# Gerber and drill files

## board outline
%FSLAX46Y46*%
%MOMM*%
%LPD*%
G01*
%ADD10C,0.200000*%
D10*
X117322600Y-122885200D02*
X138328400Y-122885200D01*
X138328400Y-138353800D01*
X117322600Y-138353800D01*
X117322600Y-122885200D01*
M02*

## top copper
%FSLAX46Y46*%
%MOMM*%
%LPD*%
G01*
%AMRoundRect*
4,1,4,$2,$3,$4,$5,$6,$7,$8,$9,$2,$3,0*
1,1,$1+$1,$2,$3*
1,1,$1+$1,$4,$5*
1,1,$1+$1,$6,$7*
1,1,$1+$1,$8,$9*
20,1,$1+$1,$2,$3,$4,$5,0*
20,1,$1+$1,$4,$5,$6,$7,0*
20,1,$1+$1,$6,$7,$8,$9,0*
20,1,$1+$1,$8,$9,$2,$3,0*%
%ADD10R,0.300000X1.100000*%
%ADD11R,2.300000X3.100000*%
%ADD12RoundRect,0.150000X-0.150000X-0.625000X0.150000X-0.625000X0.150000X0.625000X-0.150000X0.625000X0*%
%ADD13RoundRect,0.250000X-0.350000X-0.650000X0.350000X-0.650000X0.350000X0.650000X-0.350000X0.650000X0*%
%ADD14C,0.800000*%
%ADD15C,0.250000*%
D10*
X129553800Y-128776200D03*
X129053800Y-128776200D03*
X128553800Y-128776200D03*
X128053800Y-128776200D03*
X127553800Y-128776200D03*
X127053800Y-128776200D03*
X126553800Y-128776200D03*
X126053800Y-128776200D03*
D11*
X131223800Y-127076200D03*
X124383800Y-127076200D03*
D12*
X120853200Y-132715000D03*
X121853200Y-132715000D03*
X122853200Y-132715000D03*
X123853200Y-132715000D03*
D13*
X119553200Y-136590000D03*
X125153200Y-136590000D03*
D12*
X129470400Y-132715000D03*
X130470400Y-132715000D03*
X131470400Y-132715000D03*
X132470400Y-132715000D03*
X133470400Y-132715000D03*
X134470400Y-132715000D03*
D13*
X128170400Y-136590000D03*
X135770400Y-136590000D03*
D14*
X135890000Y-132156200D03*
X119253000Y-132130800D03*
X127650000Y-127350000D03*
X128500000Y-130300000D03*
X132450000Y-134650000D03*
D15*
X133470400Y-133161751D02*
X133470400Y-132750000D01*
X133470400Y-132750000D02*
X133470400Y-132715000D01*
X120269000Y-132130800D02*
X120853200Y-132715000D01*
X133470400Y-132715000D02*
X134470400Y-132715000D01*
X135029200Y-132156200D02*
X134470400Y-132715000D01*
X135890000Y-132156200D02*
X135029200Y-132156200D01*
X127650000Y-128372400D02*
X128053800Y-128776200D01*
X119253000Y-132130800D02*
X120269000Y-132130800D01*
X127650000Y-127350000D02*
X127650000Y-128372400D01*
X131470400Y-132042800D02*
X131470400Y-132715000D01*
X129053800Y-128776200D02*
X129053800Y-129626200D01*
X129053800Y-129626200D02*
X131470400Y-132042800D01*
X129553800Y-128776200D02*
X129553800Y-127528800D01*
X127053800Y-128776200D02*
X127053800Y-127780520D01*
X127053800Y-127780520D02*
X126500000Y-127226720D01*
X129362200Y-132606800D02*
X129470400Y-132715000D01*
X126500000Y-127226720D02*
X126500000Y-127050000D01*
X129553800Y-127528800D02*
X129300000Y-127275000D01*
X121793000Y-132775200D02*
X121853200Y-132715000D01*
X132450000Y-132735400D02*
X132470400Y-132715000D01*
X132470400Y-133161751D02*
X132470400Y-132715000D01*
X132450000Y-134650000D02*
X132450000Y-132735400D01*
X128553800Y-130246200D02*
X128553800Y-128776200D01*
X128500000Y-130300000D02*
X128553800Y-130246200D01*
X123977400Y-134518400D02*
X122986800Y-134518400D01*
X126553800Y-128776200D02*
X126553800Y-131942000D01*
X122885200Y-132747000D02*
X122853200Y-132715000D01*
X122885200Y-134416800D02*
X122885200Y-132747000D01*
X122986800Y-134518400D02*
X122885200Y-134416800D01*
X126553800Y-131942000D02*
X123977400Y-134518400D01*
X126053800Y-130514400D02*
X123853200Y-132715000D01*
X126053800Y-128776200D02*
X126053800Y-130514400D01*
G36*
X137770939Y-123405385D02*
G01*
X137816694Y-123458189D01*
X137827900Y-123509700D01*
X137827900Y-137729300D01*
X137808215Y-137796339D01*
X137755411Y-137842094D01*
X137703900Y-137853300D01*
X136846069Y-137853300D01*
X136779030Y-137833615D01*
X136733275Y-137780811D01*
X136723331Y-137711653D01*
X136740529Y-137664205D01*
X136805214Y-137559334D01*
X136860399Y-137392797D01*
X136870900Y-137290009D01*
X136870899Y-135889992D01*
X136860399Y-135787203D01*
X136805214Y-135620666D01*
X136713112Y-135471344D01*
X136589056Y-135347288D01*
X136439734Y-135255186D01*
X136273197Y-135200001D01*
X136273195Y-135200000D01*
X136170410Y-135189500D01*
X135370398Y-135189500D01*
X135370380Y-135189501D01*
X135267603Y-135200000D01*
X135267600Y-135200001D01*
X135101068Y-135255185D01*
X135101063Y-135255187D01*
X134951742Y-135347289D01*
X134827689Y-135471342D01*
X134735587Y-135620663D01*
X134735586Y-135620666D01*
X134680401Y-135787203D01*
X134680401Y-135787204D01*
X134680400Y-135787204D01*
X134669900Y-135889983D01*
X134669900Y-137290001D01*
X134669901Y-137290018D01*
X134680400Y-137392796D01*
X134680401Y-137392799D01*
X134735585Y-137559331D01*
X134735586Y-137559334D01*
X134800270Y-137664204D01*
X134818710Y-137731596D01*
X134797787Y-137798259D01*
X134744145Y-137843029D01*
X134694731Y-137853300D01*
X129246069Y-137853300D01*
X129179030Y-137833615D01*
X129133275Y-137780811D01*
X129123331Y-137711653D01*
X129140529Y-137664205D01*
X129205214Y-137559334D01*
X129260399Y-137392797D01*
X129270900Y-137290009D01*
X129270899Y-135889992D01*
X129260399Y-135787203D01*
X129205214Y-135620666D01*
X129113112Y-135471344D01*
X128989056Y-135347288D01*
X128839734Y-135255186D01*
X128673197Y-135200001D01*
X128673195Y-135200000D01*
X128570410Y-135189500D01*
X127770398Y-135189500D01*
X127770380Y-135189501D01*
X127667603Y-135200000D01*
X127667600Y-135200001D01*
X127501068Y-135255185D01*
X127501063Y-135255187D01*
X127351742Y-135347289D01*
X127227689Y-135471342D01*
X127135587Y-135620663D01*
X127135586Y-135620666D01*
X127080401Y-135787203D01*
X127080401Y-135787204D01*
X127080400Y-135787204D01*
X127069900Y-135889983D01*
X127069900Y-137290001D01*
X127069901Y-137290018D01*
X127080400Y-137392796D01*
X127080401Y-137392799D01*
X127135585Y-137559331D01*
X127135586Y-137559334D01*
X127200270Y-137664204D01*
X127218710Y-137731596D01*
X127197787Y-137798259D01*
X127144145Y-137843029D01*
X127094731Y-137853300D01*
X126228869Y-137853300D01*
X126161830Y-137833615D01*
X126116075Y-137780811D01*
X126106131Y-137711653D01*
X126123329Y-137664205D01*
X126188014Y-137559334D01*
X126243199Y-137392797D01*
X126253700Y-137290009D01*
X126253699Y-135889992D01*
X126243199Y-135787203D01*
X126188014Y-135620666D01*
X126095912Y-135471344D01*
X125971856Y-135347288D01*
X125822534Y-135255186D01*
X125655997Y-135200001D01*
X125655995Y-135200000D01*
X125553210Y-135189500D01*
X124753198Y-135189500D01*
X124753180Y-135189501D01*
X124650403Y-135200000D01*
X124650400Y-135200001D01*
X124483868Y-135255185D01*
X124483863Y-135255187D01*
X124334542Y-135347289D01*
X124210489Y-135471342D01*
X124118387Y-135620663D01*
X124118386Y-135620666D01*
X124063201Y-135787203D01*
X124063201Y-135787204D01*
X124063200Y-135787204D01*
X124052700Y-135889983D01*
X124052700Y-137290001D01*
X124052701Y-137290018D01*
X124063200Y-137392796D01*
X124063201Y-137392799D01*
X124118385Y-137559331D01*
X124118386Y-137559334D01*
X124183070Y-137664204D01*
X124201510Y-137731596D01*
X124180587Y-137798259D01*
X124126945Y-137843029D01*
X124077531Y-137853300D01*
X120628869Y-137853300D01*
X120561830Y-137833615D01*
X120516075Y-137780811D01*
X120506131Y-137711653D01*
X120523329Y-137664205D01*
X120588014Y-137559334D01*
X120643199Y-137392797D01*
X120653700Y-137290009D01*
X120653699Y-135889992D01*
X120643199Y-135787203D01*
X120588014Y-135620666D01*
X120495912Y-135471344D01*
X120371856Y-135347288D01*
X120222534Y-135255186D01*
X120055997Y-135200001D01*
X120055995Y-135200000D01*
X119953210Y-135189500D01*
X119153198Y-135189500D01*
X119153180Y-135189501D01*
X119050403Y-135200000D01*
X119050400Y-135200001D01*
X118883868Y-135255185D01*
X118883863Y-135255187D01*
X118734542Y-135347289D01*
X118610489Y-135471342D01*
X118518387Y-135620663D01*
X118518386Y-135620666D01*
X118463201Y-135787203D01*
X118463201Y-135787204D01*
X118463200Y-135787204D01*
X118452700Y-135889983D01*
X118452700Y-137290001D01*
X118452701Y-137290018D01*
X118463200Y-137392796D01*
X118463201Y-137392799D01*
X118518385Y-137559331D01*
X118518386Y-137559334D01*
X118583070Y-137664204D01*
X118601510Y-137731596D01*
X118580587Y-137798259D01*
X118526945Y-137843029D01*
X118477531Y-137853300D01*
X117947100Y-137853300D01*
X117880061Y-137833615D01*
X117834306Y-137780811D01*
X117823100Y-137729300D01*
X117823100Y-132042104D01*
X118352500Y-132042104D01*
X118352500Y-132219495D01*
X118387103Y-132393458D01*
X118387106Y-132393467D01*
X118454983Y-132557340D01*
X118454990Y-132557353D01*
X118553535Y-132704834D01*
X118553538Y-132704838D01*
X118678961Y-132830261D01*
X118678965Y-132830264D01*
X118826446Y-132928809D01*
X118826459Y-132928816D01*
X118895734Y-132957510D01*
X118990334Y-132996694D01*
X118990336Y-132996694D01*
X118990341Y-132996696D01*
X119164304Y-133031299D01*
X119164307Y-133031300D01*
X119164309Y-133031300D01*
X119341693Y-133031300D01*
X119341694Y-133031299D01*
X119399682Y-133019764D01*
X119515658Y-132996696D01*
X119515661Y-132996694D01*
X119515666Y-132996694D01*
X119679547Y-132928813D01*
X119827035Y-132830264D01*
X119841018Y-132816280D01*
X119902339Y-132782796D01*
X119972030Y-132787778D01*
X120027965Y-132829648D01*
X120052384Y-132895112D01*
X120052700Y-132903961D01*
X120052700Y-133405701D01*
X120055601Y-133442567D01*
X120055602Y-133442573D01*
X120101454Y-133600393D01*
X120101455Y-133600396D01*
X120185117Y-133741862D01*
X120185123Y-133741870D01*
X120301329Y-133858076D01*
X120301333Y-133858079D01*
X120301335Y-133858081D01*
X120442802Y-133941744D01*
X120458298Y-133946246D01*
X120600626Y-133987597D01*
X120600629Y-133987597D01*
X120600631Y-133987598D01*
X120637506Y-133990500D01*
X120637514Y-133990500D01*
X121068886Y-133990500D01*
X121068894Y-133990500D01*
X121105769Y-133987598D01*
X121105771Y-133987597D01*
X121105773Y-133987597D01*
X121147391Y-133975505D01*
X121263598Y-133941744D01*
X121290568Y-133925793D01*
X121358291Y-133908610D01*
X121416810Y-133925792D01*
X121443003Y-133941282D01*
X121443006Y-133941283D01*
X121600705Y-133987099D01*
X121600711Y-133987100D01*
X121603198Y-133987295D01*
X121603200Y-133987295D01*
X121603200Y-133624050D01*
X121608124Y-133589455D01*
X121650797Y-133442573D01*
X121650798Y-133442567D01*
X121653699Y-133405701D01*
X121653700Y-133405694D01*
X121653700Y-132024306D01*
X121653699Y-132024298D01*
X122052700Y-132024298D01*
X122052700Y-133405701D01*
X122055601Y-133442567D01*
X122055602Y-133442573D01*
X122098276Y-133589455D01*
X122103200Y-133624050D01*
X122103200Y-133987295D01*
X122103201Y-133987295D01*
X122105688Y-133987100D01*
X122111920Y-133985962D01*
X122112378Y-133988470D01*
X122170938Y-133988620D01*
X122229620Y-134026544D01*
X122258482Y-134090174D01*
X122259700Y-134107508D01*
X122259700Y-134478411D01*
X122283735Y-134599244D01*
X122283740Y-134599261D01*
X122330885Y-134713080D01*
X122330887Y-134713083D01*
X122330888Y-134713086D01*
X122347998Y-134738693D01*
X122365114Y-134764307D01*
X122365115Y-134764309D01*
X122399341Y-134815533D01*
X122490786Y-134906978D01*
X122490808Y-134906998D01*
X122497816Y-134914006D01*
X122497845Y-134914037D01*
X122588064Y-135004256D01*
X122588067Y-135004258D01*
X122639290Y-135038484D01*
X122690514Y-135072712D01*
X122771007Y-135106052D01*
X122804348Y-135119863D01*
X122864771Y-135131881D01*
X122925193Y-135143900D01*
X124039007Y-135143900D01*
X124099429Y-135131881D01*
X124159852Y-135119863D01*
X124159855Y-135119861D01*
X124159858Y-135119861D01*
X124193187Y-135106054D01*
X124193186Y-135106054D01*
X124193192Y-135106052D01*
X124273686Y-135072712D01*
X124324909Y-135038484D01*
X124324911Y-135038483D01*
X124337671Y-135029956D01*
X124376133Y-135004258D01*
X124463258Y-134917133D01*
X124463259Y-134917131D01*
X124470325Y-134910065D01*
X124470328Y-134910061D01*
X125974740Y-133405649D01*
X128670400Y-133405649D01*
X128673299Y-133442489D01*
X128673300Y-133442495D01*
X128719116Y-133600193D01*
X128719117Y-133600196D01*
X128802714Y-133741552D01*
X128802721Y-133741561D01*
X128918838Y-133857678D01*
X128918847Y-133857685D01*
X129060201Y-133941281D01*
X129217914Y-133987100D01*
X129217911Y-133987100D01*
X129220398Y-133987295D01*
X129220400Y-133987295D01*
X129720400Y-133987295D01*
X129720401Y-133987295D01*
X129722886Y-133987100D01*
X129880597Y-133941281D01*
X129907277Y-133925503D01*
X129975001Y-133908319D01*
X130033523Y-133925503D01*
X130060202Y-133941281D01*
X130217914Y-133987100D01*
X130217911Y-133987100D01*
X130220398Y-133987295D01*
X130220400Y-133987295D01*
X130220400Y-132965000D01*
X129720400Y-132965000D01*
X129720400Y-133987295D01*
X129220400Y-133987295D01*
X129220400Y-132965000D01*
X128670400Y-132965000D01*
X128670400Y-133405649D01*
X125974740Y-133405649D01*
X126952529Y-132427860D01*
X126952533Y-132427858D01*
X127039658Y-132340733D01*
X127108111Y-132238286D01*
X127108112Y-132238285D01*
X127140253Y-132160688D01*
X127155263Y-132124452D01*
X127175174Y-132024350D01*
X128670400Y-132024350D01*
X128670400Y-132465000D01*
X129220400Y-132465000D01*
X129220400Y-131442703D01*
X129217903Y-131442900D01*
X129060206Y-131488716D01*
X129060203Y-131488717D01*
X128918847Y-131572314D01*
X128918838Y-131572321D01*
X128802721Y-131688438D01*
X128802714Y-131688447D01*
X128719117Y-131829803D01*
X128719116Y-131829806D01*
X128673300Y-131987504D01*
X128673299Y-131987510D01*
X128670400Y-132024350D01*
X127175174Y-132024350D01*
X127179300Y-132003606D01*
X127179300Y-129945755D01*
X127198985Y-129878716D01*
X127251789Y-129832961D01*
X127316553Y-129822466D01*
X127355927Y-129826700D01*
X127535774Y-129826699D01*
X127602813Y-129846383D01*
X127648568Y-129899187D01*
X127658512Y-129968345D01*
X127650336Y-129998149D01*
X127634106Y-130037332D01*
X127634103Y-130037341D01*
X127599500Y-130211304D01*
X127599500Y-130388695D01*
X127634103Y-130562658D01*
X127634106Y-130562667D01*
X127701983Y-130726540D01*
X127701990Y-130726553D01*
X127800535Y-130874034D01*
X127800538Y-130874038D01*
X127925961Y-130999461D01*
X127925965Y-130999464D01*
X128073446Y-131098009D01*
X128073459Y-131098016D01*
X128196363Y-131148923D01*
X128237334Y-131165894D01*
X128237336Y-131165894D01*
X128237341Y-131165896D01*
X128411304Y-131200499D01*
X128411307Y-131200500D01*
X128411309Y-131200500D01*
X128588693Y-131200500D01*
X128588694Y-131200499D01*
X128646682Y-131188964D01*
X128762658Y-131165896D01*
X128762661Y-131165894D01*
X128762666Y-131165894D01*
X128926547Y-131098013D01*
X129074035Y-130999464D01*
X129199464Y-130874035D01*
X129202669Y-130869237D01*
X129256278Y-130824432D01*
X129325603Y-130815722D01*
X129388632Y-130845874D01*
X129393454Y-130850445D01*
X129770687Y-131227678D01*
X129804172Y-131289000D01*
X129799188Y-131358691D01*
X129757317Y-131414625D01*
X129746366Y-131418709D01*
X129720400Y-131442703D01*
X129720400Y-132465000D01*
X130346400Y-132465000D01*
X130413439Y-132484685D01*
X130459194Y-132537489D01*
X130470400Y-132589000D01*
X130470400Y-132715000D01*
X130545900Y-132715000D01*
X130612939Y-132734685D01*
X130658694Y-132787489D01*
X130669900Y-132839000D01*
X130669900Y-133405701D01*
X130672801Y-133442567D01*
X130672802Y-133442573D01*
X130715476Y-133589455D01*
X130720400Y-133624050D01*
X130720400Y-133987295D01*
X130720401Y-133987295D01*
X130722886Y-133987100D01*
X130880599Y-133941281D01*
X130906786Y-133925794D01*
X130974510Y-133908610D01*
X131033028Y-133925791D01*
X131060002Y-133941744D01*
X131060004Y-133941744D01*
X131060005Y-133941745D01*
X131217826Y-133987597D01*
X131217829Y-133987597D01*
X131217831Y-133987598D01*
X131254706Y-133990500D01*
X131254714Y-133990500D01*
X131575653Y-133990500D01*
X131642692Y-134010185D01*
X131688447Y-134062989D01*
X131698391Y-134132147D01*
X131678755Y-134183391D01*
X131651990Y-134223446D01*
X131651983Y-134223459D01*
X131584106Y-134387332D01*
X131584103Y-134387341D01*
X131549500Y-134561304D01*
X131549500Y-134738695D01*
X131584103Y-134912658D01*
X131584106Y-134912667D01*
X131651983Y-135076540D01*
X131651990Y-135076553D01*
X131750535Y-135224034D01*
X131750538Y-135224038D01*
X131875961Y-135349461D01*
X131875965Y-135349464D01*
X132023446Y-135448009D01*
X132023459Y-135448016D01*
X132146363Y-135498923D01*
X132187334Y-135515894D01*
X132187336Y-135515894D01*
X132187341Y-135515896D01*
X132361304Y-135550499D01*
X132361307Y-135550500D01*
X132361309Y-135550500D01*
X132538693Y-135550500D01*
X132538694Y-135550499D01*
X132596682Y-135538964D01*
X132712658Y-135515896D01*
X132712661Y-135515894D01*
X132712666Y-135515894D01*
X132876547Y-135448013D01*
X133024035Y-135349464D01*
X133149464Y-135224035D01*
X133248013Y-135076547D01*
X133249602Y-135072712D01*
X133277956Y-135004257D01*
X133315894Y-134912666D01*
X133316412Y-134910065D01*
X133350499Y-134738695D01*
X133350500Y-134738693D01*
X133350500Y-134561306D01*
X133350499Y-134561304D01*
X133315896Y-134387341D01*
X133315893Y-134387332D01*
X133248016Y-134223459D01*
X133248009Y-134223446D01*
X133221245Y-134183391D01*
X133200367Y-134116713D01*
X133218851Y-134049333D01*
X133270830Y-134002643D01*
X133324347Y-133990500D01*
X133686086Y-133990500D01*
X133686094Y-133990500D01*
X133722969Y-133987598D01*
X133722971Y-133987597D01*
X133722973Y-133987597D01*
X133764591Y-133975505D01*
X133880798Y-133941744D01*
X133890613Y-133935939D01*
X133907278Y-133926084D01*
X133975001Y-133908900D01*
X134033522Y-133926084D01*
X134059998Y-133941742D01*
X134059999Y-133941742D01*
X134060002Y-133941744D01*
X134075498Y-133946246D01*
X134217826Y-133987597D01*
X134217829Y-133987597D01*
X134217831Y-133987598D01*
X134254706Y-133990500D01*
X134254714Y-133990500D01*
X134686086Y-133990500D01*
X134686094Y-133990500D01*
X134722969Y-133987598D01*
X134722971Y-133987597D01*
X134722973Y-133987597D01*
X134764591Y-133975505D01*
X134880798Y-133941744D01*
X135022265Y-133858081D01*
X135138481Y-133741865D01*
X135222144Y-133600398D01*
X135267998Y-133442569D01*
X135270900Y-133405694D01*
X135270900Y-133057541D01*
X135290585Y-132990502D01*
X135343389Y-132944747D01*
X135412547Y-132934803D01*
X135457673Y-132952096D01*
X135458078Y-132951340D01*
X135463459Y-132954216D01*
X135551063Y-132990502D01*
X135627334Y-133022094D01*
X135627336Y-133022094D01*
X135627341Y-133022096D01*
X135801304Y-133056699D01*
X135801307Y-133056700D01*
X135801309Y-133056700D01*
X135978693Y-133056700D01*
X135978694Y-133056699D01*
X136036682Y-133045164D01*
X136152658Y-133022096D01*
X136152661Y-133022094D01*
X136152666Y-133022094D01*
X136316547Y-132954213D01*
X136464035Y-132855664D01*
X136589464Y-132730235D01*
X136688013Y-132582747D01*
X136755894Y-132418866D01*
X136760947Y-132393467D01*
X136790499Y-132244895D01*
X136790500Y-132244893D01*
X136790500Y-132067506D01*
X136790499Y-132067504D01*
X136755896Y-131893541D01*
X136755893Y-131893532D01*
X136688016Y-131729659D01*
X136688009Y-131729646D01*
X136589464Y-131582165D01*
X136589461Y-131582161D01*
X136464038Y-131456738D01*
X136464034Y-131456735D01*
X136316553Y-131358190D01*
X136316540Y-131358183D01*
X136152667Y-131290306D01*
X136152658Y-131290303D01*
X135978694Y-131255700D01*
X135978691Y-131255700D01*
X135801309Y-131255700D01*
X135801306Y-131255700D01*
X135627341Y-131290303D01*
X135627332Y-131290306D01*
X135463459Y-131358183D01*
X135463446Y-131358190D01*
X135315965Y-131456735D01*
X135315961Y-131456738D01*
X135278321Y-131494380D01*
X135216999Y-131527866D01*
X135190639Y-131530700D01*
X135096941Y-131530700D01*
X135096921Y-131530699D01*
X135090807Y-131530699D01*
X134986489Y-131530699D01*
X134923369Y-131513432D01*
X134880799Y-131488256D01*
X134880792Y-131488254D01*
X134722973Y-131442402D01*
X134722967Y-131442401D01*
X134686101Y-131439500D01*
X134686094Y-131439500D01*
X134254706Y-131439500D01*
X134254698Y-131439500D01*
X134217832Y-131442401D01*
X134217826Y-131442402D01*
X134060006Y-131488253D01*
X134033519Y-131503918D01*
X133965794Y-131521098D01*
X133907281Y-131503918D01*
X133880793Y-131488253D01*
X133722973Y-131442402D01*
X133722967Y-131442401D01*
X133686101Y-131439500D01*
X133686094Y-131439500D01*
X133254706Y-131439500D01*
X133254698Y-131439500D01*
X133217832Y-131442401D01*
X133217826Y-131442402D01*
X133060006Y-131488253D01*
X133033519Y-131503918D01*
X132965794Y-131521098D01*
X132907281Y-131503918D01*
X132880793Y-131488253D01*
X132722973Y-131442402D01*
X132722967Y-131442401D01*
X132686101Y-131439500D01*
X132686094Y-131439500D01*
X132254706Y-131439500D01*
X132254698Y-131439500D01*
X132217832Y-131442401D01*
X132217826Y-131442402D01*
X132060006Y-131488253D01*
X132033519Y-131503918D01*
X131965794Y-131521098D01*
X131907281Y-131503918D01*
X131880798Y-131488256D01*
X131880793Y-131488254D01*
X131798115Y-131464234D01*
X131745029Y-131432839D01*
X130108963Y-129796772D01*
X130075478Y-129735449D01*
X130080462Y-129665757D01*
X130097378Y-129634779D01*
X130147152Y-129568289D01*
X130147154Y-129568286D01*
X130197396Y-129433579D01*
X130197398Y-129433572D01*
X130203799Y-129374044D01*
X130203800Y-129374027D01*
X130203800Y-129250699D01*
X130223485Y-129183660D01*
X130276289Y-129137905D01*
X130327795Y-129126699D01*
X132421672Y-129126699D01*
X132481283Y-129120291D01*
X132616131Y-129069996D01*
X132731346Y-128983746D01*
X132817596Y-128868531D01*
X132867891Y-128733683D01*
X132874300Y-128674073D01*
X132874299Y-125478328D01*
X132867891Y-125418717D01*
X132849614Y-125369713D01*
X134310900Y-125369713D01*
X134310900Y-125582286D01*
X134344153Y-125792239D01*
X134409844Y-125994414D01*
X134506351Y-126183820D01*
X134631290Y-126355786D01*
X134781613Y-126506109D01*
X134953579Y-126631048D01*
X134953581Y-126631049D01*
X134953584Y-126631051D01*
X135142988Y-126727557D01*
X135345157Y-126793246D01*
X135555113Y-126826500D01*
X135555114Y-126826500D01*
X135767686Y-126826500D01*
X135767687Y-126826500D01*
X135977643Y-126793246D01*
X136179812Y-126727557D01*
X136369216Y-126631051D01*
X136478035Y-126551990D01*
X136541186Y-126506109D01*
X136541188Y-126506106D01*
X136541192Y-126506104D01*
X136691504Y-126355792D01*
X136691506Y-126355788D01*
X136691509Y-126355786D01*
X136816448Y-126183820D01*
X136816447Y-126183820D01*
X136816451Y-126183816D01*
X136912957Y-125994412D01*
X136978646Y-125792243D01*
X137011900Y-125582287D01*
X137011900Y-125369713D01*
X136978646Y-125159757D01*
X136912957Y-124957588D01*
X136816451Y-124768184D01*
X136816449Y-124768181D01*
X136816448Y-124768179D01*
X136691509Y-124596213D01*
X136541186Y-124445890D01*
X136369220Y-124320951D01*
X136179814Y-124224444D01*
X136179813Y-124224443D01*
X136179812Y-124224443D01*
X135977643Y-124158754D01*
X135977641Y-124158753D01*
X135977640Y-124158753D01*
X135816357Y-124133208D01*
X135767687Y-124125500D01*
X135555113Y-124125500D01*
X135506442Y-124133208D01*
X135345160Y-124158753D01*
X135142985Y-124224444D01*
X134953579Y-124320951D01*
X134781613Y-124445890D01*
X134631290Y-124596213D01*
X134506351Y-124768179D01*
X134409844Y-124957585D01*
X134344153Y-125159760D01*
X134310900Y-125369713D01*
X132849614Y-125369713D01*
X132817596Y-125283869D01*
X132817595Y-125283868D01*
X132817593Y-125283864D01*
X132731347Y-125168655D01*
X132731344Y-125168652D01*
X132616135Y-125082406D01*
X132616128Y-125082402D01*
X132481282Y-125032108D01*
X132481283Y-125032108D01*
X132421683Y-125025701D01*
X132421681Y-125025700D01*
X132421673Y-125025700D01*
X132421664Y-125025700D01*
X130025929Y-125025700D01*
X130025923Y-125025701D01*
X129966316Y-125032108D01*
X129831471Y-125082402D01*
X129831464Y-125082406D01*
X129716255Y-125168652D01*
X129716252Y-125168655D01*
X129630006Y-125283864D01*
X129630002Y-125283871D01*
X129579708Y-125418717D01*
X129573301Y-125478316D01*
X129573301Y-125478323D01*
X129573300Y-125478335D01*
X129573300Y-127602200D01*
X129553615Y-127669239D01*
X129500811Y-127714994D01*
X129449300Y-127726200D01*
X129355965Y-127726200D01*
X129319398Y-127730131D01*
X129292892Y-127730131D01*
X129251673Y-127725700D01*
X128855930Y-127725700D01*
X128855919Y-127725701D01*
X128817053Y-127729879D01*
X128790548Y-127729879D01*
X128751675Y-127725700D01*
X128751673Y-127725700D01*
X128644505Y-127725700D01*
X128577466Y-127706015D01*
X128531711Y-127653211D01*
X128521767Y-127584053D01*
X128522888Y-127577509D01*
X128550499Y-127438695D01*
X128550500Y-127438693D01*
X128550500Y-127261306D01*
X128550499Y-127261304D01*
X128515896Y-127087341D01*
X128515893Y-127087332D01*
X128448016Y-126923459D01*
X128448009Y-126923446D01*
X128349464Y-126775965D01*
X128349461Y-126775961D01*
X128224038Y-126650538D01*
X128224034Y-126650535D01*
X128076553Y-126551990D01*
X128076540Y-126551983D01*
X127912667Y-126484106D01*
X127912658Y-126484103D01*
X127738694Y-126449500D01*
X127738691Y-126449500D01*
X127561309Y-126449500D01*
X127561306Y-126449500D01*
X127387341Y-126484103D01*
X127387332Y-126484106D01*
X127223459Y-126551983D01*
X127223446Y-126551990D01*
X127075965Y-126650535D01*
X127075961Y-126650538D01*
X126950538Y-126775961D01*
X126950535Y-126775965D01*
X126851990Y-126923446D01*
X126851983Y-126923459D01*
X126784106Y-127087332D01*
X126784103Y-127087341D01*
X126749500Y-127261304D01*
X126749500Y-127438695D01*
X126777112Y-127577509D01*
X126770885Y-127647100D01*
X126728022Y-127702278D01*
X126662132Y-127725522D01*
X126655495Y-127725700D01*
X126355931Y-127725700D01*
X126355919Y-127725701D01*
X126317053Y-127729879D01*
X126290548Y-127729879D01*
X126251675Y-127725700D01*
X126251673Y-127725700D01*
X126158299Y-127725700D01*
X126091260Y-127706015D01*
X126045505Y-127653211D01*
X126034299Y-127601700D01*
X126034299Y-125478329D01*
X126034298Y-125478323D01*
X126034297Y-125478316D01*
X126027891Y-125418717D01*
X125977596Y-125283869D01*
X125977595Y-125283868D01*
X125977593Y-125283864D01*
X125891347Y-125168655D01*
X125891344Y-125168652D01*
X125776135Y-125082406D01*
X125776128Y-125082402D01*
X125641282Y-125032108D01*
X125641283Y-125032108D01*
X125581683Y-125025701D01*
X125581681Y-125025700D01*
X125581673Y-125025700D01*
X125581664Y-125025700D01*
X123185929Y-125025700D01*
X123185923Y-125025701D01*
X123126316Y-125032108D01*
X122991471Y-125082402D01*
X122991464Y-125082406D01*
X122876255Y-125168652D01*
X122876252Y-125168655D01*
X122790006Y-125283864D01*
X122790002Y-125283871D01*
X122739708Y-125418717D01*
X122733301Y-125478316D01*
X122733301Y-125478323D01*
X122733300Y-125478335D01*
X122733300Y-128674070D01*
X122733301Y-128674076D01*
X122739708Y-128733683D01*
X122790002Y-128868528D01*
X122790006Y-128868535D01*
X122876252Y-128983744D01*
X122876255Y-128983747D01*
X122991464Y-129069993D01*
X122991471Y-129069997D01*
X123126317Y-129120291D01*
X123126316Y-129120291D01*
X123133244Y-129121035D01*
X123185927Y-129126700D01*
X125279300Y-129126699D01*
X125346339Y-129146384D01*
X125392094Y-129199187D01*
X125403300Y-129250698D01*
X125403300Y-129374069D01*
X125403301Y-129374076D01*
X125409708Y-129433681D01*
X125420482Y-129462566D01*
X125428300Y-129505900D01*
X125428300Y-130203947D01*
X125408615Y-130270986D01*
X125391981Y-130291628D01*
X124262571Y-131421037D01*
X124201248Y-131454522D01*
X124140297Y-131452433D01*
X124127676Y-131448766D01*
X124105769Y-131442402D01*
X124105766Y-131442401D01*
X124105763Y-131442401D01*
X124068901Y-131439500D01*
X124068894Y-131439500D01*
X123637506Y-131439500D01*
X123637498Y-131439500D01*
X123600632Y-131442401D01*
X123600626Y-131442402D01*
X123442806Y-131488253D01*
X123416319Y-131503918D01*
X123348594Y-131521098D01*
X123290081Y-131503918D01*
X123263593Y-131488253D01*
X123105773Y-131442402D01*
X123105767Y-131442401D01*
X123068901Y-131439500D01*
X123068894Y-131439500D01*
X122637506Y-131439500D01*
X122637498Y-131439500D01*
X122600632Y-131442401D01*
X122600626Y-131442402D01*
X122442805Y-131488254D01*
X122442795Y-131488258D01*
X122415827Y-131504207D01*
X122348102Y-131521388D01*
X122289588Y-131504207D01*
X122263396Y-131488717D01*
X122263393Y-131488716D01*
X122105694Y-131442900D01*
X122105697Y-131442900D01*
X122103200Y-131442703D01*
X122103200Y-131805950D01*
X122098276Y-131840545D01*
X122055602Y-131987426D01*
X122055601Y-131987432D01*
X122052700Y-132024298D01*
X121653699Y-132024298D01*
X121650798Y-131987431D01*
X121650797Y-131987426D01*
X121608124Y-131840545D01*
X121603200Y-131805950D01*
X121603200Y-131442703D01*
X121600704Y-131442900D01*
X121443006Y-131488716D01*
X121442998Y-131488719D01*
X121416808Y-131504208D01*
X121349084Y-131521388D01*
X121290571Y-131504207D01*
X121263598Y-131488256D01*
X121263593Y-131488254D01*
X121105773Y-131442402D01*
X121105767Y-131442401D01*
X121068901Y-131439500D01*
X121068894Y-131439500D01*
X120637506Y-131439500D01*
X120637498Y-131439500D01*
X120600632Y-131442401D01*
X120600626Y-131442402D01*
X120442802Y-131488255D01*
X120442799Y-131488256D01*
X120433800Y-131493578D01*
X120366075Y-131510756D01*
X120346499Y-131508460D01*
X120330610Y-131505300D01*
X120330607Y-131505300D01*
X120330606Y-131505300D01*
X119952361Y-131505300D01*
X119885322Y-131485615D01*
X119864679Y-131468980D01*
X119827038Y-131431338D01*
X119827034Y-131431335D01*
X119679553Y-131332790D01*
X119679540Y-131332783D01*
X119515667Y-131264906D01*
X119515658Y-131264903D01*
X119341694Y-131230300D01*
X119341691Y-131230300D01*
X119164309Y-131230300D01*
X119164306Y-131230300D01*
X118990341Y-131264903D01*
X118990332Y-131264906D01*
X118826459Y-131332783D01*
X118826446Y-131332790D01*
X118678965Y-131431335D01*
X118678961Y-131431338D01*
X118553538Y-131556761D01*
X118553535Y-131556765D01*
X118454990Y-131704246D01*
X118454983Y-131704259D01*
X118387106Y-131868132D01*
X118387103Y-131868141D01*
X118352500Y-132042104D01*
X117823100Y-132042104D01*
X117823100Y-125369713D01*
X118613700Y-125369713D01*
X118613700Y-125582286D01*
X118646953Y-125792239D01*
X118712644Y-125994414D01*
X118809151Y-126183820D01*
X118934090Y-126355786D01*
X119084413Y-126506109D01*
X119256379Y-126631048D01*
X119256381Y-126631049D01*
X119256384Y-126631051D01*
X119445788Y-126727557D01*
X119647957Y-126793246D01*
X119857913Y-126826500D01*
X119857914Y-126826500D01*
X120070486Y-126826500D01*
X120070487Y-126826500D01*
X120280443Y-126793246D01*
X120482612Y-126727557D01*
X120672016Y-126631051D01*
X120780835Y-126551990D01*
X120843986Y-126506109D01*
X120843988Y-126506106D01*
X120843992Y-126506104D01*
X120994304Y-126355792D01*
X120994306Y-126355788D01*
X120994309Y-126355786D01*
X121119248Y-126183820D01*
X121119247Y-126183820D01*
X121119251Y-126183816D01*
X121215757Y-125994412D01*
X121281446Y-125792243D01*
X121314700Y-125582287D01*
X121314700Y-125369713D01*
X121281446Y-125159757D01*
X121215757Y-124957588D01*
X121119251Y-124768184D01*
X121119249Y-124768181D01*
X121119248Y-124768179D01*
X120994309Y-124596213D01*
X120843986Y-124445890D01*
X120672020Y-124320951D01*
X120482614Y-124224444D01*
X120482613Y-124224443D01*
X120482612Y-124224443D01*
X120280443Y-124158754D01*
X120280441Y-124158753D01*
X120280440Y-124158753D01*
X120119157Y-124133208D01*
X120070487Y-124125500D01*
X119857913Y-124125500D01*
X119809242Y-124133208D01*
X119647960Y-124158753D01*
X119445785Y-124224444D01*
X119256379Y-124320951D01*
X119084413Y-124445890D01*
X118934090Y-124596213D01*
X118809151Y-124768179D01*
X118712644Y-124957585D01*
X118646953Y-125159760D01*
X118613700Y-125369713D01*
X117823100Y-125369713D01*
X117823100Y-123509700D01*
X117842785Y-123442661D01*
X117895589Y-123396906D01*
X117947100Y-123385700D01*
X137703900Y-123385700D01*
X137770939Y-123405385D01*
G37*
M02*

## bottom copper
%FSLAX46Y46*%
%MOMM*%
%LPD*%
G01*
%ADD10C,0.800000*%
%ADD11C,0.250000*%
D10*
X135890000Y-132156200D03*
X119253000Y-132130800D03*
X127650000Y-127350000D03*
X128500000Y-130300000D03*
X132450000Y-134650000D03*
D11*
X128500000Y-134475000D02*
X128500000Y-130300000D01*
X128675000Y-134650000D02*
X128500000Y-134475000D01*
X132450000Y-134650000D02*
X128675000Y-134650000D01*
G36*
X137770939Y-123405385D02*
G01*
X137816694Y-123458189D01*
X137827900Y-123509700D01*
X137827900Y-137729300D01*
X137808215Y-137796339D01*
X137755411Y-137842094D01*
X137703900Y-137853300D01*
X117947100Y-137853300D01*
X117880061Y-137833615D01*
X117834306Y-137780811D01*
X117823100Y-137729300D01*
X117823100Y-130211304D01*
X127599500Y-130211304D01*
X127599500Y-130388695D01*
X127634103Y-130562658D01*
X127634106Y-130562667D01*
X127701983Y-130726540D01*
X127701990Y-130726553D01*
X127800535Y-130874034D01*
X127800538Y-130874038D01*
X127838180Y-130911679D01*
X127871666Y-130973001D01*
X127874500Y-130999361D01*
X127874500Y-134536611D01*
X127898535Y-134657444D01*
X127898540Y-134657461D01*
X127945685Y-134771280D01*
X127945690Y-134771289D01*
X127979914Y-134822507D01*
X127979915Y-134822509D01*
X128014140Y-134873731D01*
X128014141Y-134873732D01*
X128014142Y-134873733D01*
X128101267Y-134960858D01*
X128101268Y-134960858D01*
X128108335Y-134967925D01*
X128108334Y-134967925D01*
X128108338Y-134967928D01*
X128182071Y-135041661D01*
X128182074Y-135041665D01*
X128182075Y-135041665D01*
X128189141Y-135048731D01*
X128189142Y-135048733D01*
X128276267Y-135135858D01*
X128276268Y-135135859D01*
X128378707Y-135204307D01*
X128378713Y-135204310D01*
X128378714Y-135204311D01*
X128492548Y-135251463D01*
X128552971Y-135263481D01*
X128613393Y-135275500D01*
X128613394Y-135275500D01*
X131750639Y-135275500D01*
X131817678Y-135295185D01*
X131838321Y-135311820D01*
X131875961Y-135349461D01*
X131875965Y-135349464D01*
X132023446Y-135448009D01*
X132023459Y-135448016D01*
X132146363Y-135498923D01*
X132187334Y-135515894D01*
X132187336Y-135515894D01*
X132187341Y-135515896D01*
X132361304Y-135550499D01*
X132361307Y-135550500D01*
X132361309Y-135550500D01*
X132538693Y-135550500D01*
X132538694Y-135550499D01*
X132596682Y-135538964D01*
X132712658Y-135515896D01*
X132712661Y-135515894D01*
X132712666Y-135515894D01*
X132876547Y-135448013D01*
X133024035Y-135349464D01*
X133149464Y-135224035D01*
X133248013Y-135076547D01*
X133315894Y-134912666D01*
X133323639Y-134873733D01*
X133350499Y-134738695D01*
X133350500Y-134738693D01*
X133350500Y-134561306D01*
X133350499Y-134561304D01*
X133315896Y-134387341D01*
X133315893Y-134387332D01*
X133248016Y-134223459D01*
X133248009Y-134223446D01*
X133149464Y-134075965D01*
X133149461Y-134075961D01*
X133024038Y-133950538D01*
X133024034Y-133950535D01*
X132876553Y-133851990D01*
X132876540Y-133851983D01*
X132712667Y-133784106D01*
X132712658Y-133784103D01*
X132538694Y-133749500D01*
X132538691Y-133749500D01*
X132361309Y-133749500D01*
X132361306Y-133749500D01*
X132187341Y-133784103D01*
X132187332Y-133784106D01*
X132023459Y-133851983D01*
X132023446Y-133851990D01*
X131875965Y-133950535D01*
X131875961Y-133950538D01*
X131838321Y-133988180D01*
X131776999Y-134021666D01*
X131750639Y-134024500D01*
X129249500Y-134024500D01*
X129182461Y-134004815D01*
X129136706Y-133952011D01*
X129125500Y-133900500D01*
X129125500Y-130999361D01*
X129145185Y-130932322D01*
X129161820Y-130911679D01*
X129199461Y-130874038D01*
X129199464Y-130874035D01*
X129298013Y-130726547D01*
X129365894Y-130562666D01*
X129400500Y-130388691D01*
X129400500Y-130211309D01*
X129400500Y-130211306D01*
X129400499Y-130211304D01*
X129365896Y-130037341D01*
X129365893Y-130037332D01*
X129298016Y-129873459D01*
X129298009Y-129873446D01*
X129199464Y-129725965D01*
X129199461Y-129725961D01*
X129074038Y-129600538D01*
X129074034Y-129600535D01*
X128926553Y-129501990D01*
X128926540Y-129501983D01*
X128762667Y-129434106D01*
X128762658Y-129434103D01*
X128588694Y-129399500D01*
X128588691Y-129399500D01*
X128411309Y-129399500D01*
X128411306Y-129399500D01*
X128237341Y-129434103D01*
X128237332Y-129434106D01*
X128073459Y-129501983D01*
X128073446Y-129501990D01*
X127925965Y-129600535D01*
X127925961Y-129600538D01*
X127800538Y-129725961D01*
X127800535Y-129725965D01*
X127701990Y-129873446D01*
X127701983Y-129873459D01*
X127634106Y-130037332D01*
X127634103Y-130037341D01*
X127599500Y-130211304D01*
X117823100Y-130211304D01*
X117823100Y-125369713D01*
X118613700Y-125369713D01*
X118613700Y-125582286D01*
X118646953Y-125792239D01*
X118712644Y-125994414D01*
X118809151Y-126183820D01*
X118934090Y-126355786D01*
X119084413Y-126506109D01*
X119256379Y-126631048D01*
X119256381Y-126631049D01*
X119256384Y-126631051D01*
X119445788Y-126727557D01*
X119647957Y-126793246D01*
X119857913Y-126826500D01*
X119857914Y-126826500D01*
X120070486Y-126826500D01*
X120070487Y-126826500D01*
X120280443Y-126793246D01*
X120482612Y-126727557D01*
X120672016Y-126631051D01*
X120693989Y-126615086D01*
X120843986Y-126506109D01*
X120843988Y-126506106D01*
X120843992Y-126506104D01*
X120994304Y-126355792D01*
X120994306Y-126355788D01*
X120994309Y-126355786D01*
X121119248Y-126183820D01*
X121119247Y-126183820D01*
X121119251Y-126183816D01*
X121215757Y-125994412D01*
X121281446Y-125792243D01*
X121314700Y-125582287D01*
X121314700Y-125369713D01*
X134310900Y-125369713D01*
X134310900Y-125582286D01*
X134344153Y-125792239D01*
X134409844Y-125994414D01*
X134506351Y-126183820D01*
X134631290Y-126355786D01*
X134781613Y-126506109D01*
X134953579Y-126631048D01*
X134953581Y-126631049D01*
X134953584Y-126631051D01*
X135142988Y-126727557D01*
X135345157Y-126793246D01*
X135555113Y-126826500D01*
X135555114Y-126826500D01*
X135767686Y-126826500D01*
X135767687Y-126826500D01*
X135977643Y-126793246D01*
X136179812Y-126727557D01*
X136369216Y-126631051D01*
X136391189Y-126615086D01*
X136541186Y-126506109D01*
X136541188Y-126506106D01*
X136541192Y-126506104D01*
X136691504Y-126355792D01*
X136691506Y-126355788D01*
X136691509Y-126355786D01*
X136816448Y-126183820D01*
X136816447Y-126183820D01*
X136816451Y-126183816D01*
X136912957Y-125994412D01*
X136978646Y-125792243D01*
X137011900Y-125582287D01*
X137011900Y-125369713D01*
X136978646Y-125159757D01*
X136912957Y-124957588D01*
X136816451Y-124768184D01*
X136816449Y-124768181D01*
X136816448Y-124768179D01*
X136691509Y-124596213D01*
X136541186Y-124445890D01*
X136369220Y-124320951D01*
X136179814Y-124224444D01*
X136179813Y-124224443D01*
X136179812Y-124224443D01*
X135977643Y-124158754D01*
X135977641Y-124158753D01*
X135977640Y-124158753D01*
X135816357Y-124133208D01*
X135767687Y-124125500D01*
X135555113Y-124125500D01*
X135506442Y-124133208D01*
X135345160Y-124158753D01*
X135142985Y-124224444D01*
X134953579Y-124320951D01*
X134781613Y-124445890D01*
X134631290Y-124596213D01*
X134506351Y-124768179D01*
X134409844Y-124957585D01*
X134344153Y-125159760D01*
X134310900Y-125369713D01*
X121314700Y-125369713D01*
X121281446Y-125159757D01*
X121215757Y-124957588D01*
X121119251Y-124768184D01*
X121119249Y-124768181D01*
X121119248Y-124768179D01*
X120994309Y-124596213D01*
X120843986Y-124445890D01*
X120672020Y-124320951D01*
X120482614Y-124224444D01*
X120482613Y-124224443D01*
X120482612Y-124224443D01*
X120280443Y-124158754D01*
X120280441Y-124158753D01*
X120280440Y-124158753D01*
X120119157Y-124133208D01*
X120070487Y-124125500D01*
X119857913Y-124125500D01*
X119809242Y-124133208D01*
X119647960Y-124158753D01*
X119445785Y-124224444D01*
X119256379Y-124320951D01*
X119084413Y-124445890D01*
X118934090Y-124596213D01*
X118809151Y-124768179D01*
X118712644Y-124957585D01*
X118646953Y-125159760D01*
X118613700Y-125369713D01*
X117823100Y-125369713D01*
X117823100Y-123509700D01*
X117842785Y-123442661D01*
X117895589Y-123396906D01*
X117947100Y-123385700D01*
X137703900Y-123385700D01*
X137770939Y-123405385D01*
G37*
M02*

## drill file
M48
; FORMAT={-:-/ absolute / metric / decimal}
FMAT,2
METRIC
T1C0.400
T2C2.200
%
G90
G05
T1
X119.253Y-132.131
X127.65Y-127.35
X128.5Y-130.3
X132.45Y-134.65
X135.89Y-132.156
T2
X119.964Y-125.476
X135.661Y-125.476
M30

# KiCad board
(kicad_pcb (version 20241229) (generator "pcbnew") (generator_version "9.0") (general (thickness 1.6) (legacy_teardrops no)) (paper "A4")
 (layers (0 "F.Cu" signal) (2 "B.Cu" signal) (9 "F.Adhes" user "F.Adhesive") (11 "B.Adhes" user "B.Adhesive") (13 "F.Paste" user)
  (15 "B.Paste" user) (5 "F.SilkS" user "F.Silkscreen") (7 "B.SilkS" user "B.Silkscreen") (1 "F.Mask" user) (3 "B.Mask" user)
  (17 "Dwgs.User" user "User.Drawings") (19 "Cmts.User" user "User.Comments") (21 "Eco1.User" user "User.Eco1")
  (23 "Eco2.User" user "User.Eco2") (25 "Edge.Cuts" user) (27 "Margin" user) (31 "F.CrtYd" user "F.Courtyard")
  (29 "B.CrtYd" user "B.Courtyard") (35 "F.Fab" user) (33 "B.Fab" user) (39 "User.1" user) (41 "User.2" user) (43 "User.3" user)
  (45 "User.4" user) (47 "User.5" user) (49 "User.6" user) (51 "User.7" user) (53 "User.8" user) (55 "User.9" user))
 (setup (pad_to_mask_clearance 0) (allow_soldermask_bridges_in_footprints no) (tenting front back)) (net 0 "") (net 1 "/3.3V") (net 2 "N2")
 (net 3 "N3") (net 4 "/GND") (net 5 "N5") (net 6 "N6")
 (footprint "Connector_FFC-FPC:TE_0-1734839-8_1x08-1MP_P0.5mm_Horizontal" (layer "F.Cu") (at 127.8038 127.4262 180)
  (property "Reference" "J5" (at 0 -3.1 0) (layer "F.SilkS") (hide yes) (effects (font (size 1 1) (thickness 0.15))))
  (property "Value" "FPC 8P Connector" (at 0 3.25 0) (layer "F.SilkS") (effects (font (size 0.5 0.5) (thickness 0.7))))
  (pad "1" smd rect (at -1.75 -1.35 180) (size 0.3 1.1) (layers "F.Cu" "F.Mask" "F.Paste") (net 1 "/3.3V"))
  (pad "2" smd rect (at -1.25 -1.35 180) (size 0.3 1.1) (layers "F.Cu" "F.Mask" "F.Paste") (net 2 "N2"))
  (pad "3" smd rect (at -0.75 -1.35 180) (size 0.3 1.1) (layers "F.Cu" "F.Mask" "F.Paste") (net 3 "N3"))
  (pad "4" smd rect (at -0.25 -1.35 180) (size 0.3 1.1) (layers "F.Cu" "F.Mask" "F.Paste") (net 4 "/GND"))
  (pad "5" smd rect (at 0.25 -1.35 180) (size 0.3 1.1) (layers "F.Cu" "F.Mask" "F.Paste") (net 4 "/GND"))
  (pad "6" smd rect (at 0.75 -1.35 180) (size 0.3 1.1) (layers "F.Cu" "F.Mask" "F.Paste") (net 1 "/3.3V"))
  (pad "7" smd rect (at 1.25 -1.35 180) (size 0.3 1.1) (layers "F.Cu" "F.Mask" "F.Paste") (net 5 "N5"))
  (pad "8" smd rect (at 1.75 -1.35 180) (size 0.3 1.1) (layers "F.Cu" "F.Mask" "F.Paste") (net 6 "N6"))
  (pad "MP" smd rect (at -3.42 0.35 180) (size 2.3 3.1) (layers "F.Cu" "F.Mask" "F.Paste"))
  (pad "MP" smd rect (at 3.42 0.35 180) (size 2.3 3.1) (layers "F.Cu" "F.Mask" "F.Paste")))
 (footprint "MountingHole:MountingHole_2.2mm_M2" (layer "F.Cu") (at 119.9642 125.476)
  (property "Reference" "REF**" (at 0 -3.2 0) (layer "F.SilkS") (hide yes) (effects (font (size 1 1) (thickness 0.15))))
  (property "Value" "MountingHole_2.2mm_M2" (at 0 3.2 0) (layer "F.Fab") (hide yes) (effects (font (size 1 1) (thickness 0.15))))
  (pad "" np_thru_hole circle (at 0 0) (size 2.2 2.2) (drill 2.2) (layers "*.Cu" "*.Mask")))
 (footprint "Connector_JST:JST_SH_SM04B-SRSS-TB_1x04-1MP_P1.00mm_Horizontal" (layer "F.Cu") (at 122.3532 134.715)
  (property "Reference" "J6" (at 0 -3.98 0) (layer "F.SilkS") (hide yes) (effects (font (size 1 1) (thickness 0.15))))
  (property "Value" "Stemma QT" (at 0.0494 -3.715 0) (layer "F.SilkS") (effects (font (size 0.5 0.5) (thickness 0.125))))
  (pad "1" smd roundrect (at -1.5 -2) (size 0.6 1.55) (layers "F.Cu" "F.Mask" "F.Paste") (roundrect_rratio 0.25) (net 4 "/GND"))
  (pad "2" smd roundrect (at -0.5 -2) (size 0.6 1.55) (layers "F.Cu" "F.Mask" "F.Paste") (roundrect_rratio 0.25) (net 1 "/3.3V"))
  (pad "3" smd roundrect (at 0.5 -2) (size 0.6 1.55) (layers "F.Cu" "F.Mask" "F.Paste") (roundrect_rratio 0.25) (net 5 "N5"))
  (pad "4" smd roundrect (at 1.5 -2) (size 0.6 1.55) (layers "F.Cu" "F.Mask" "F.Paste") (roundrect_rratio 0.25) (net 6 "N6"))
  (pad "MP" smd roundrect (at -2.8 1.875) (size 1.2 1.8) (layers "F.Cu" "F.Mask" "F.Paste") (roundrect_rratio 0.2083333333))
  (pad "MP" smd roundrect (at 2.8 1.875) (size 1.2 1.8) (layers "F.Cu" "F.Mask" "F.Paste") (roundrect_rratio 0.2083333333)))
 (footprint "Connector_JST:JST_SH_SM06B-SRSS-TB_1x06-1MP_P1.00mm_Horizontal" (layer "F.Cu") (at 131.9704 134.715)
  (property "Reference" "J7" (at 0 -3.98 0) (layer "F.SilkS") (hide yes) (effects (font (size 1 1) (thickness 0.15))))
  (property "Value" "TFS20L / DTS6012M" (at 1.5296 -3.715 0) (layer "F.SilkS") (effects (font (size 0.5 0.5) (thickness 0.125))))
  (pad "1" smd roundrect (at -2.5 -2) (size 0.6 1.55) (layers "F.Cu" "F.Mask" "F.Paste") (roundrect_rratio 0.25) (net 1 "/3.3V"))
  (pad "2" smd roundrect (at -1.5 -2) (size 0.6 1.55) (layers "F.Cu" "F.Mask" "F.Paste") (roundrect_rratio 0.25) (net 1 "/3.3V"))
  (pad "3" smd roundrect (at -0.5 -2) (size 0.6 1.55) (layers "F.Cu" "F.Mask" "F.Paste") (roundrect_rratio 0.25) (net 2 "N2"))
  (pad "4" smd roundrect (at 0.5 -2) (size 0.6 1.55) (layers "F.Cu" "F.Mask" "F.Paste") (roundrect_rratio 0.25) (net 3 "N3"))
  (pad "5" smd roundrect (at 1.5 -2) (size 0.6 1.55) (layers "F.Cu" "F.Mask" "F.Paste") (roundrect_rratio 0.25) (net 4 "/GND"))
  (pad "6" smd roundrect (at 2.5 -2) (size 0.6 1.55) (layers "F.Cu" "F.Mask" "F.Paste") (roundrect_rratio 0.25) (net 4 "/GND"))
  (pad "MP" smd roundrect (at -3.8 1.875) (size 1.2 1.8) (layers "F.Cu" "F.Mask" "F.Paste") (roundrect_rratio 0.2083333333))
  (pad "MP" smd roundrect (at 3.8 1.875) (size 1.2 1.8) (layers "F.Cu" "F.Mask" "F.Paste") (roundrect_rratio 0.2083333333)))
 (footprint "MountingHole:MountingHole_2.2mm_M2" (layer "F.Cu") (at 135.6614 125.476)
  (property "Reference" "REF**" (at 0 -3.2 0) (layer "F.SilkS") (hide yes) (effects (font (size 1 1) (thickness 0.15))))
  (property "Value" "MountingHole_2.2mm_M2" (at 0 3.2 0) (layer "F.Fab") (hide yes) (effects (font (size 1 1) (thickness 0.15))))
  (pad "" np_thru_hole circle (at 0 0) (size 2.2 2.2) (drill 2.2) (layers "*.Cu" "*.Mask")))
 (gr_rect (start 117.3226 122.8852) (end 138.3284 138.3538) (stroke (width 0.2) (type default)) (fill no) (layer "Edge.Cuts"))
 (segment (start 133.4704 133.161751) (end 133.4704 132.75) (width 0.25) (layer "F.Cu") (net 4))
 (segment (start 133.4704 132.75) (end 133.4704 132.715) (width 0.25) (layer "F.Cu") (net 4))
 (segment (start 120.269 132.1308) (end 120.8532 132.715) (width 0.25) (layer "F.Cu") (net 4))
 (segment (start 133.4704 132.715) (end 134.4704 132.715) (width 0.25) (layer "F.Cu") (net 4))
 (segment (start 135.0292 132.1562) (end 134.4704 132.715) (width 0.25) (layer "F.Cu") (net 4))
 (segment (start 135.89 132.1562) (end 135.0292 132.1562) (width 0.25) (layer "F.Cu") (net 4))
 (segment (start 127.65 128.3724) (end 128.0538 128.7762) (width 0.25) (layer "F.Cu") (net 4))
 (segment (start 119.253 132.1308) (end 120.269 132.1308) (width 0.25) (layer "F.Cu") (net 4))
 (segment (start 127.65 127.35) (end 127.65 128.3724) (width 0.25) (layer "F.Cu") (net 4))
 (via (at 135.89 132.1562) (size 0.8) (drill 0.4) (layers "F.Cu" "B.Cu") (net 4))
 (via (at 119.253 132.1308) (size 0.8) (drill 0.4) (layers "F.Cu" "B.Cu") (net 4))
 (via (at 127.65 127.35) (size 0.8) (drill 0.4) (layers "F.Cu" "B.Cu") (free yes) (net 4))
 (segment (start 131.4704 132.0428) (end 131.4704 132.715) (width 0.25) (layer "F.Cu") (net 2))
 (segment (start 129.0538 128.7762) (end 129.0538 129.6262) (width 0.25) (layer "F.Cu") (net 2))
 (segment (start 129.0538 129.6262) (end 131.4704 132.0428) (width 0.25) (layer "F.Cu") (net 2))
 (segment (start 129.5538 128.7762) (end 129.5538 127.5288) (width 0.25) (layer "F.Cu") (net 1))
 (segment (start 127.0538 128.7762) (end 127.0538 127.78052) (width 0.25) (layer "F.Cu") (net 1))
 (segment (start 127.0538 127.78052) (end 126.5 127.22672) (width 0.25) (layer "F.Cu") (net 1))
 (segment (start 129.3622 132.6068) (end 129.4704 132.715) (width 0.25) (layer "F.Cu") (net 1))
 (segment (start 126.5 127.22672) (end 126.5 127.05) (width 0.25) (layer "F.Cu") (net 1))
 (segment (start 129.5538 127.5288) (end 129.3 127.275) (width 0.25) (layer "F.Cu") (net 1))
 (segment (start 121.793 132.7752) (end 121.8532 132.715) (width 0.25) (layer "F.Cu") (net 1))
 (segment (start 132.45 132.7354) (end 132.4704 132.715) (width 0.25) (layer "F.Cu") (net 3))
 (segment (start 132.4704 133.161751) (end 132.4704 132.715) (width 0.25) (layer "F.Cu") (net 3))
 (segment (start 132.45 134.65) (end 132.45 132.7354) (width 0.25) (layer "F.Cu") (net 3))
 (segment (start 128.5538 130.2462) (end 128.5538 128.7762) (width 0.25) (layer "F.Cu") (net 3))
 (segment (start 128.5 130.3) (end 128.5538 130.2462) (width 0.25) (layer "F.Cu") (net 3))
 (via (at 128.5 130.3) (size 0.8) (drill 0.4) (layers "F.Cu" "B.Cu") (free yes) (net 3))
 (via (at 132.45 134.65) (size 0.8) (drill 0.4) (layers "F.Cu" "B.Cu") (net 3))
 (segment (start 128.5 134.475) (end 128.5 130.3) (width 0.25) (layer "B.Cu") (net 3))
 (segment (start 128.675 134.65) (end 128.5 134.475) (width 0.25) (layer "B.Cu") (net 3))
 (segment (start 132.45 134.65) (end 128.675 134.65) (width 0.25) (layer "B.Cu") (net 3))
 (segment (start 123.9774 134.5184) (end 122.9868 134.5184) (width 0.25) (layer "F.Cu") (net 5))
 (segment (start 126.5538 128.7762) (end 126.5538 131.942) (width 0.25) (layer "F.Cu") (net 5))
 (segment (start 122.8852 132.747) (end 122.8532 132.715) (width 0.25) (layer "F.Cu") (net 5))
 (segment (start 122.8852 134.4168) (end 122.8852 132.747) (width 0.25) (layer "F.Cu") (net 5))
 (segment (start 122.9868 134.5184) (end 122.8852 134.4168) (width 0.25) (layer "F.Cu") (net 5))
 (segment (start 126.5538 131.942) (end 123.9774 134.5184) (width 0.25) (layer "F.Cu") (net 5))
 (segment (start 126.0538 130.5144) (end 123.8532 132.715) (width 0.25) (layer "F.Cu") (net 6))
 (segment (start 126.0538 128.7762) (end 126.0538 130.5144) (width 0.25) (layer "F.Cu") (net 6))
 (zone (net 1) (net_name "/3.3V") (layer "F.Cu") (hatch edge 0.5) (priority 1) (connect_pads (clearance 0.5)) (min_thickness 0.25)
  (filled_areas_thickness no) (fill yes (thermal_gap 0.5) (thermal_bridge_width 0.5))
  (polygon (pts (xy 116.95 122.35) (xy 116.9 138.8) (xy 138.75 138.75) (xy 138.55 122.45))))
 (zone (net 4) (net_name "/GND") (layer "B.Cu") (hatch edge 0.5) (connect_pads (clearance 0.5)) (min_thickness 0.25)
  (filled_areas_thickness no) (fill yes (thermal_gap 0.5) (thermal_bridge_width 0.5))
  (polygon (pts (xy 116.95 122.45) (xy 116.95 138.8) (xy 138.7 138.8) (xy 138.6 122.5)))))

